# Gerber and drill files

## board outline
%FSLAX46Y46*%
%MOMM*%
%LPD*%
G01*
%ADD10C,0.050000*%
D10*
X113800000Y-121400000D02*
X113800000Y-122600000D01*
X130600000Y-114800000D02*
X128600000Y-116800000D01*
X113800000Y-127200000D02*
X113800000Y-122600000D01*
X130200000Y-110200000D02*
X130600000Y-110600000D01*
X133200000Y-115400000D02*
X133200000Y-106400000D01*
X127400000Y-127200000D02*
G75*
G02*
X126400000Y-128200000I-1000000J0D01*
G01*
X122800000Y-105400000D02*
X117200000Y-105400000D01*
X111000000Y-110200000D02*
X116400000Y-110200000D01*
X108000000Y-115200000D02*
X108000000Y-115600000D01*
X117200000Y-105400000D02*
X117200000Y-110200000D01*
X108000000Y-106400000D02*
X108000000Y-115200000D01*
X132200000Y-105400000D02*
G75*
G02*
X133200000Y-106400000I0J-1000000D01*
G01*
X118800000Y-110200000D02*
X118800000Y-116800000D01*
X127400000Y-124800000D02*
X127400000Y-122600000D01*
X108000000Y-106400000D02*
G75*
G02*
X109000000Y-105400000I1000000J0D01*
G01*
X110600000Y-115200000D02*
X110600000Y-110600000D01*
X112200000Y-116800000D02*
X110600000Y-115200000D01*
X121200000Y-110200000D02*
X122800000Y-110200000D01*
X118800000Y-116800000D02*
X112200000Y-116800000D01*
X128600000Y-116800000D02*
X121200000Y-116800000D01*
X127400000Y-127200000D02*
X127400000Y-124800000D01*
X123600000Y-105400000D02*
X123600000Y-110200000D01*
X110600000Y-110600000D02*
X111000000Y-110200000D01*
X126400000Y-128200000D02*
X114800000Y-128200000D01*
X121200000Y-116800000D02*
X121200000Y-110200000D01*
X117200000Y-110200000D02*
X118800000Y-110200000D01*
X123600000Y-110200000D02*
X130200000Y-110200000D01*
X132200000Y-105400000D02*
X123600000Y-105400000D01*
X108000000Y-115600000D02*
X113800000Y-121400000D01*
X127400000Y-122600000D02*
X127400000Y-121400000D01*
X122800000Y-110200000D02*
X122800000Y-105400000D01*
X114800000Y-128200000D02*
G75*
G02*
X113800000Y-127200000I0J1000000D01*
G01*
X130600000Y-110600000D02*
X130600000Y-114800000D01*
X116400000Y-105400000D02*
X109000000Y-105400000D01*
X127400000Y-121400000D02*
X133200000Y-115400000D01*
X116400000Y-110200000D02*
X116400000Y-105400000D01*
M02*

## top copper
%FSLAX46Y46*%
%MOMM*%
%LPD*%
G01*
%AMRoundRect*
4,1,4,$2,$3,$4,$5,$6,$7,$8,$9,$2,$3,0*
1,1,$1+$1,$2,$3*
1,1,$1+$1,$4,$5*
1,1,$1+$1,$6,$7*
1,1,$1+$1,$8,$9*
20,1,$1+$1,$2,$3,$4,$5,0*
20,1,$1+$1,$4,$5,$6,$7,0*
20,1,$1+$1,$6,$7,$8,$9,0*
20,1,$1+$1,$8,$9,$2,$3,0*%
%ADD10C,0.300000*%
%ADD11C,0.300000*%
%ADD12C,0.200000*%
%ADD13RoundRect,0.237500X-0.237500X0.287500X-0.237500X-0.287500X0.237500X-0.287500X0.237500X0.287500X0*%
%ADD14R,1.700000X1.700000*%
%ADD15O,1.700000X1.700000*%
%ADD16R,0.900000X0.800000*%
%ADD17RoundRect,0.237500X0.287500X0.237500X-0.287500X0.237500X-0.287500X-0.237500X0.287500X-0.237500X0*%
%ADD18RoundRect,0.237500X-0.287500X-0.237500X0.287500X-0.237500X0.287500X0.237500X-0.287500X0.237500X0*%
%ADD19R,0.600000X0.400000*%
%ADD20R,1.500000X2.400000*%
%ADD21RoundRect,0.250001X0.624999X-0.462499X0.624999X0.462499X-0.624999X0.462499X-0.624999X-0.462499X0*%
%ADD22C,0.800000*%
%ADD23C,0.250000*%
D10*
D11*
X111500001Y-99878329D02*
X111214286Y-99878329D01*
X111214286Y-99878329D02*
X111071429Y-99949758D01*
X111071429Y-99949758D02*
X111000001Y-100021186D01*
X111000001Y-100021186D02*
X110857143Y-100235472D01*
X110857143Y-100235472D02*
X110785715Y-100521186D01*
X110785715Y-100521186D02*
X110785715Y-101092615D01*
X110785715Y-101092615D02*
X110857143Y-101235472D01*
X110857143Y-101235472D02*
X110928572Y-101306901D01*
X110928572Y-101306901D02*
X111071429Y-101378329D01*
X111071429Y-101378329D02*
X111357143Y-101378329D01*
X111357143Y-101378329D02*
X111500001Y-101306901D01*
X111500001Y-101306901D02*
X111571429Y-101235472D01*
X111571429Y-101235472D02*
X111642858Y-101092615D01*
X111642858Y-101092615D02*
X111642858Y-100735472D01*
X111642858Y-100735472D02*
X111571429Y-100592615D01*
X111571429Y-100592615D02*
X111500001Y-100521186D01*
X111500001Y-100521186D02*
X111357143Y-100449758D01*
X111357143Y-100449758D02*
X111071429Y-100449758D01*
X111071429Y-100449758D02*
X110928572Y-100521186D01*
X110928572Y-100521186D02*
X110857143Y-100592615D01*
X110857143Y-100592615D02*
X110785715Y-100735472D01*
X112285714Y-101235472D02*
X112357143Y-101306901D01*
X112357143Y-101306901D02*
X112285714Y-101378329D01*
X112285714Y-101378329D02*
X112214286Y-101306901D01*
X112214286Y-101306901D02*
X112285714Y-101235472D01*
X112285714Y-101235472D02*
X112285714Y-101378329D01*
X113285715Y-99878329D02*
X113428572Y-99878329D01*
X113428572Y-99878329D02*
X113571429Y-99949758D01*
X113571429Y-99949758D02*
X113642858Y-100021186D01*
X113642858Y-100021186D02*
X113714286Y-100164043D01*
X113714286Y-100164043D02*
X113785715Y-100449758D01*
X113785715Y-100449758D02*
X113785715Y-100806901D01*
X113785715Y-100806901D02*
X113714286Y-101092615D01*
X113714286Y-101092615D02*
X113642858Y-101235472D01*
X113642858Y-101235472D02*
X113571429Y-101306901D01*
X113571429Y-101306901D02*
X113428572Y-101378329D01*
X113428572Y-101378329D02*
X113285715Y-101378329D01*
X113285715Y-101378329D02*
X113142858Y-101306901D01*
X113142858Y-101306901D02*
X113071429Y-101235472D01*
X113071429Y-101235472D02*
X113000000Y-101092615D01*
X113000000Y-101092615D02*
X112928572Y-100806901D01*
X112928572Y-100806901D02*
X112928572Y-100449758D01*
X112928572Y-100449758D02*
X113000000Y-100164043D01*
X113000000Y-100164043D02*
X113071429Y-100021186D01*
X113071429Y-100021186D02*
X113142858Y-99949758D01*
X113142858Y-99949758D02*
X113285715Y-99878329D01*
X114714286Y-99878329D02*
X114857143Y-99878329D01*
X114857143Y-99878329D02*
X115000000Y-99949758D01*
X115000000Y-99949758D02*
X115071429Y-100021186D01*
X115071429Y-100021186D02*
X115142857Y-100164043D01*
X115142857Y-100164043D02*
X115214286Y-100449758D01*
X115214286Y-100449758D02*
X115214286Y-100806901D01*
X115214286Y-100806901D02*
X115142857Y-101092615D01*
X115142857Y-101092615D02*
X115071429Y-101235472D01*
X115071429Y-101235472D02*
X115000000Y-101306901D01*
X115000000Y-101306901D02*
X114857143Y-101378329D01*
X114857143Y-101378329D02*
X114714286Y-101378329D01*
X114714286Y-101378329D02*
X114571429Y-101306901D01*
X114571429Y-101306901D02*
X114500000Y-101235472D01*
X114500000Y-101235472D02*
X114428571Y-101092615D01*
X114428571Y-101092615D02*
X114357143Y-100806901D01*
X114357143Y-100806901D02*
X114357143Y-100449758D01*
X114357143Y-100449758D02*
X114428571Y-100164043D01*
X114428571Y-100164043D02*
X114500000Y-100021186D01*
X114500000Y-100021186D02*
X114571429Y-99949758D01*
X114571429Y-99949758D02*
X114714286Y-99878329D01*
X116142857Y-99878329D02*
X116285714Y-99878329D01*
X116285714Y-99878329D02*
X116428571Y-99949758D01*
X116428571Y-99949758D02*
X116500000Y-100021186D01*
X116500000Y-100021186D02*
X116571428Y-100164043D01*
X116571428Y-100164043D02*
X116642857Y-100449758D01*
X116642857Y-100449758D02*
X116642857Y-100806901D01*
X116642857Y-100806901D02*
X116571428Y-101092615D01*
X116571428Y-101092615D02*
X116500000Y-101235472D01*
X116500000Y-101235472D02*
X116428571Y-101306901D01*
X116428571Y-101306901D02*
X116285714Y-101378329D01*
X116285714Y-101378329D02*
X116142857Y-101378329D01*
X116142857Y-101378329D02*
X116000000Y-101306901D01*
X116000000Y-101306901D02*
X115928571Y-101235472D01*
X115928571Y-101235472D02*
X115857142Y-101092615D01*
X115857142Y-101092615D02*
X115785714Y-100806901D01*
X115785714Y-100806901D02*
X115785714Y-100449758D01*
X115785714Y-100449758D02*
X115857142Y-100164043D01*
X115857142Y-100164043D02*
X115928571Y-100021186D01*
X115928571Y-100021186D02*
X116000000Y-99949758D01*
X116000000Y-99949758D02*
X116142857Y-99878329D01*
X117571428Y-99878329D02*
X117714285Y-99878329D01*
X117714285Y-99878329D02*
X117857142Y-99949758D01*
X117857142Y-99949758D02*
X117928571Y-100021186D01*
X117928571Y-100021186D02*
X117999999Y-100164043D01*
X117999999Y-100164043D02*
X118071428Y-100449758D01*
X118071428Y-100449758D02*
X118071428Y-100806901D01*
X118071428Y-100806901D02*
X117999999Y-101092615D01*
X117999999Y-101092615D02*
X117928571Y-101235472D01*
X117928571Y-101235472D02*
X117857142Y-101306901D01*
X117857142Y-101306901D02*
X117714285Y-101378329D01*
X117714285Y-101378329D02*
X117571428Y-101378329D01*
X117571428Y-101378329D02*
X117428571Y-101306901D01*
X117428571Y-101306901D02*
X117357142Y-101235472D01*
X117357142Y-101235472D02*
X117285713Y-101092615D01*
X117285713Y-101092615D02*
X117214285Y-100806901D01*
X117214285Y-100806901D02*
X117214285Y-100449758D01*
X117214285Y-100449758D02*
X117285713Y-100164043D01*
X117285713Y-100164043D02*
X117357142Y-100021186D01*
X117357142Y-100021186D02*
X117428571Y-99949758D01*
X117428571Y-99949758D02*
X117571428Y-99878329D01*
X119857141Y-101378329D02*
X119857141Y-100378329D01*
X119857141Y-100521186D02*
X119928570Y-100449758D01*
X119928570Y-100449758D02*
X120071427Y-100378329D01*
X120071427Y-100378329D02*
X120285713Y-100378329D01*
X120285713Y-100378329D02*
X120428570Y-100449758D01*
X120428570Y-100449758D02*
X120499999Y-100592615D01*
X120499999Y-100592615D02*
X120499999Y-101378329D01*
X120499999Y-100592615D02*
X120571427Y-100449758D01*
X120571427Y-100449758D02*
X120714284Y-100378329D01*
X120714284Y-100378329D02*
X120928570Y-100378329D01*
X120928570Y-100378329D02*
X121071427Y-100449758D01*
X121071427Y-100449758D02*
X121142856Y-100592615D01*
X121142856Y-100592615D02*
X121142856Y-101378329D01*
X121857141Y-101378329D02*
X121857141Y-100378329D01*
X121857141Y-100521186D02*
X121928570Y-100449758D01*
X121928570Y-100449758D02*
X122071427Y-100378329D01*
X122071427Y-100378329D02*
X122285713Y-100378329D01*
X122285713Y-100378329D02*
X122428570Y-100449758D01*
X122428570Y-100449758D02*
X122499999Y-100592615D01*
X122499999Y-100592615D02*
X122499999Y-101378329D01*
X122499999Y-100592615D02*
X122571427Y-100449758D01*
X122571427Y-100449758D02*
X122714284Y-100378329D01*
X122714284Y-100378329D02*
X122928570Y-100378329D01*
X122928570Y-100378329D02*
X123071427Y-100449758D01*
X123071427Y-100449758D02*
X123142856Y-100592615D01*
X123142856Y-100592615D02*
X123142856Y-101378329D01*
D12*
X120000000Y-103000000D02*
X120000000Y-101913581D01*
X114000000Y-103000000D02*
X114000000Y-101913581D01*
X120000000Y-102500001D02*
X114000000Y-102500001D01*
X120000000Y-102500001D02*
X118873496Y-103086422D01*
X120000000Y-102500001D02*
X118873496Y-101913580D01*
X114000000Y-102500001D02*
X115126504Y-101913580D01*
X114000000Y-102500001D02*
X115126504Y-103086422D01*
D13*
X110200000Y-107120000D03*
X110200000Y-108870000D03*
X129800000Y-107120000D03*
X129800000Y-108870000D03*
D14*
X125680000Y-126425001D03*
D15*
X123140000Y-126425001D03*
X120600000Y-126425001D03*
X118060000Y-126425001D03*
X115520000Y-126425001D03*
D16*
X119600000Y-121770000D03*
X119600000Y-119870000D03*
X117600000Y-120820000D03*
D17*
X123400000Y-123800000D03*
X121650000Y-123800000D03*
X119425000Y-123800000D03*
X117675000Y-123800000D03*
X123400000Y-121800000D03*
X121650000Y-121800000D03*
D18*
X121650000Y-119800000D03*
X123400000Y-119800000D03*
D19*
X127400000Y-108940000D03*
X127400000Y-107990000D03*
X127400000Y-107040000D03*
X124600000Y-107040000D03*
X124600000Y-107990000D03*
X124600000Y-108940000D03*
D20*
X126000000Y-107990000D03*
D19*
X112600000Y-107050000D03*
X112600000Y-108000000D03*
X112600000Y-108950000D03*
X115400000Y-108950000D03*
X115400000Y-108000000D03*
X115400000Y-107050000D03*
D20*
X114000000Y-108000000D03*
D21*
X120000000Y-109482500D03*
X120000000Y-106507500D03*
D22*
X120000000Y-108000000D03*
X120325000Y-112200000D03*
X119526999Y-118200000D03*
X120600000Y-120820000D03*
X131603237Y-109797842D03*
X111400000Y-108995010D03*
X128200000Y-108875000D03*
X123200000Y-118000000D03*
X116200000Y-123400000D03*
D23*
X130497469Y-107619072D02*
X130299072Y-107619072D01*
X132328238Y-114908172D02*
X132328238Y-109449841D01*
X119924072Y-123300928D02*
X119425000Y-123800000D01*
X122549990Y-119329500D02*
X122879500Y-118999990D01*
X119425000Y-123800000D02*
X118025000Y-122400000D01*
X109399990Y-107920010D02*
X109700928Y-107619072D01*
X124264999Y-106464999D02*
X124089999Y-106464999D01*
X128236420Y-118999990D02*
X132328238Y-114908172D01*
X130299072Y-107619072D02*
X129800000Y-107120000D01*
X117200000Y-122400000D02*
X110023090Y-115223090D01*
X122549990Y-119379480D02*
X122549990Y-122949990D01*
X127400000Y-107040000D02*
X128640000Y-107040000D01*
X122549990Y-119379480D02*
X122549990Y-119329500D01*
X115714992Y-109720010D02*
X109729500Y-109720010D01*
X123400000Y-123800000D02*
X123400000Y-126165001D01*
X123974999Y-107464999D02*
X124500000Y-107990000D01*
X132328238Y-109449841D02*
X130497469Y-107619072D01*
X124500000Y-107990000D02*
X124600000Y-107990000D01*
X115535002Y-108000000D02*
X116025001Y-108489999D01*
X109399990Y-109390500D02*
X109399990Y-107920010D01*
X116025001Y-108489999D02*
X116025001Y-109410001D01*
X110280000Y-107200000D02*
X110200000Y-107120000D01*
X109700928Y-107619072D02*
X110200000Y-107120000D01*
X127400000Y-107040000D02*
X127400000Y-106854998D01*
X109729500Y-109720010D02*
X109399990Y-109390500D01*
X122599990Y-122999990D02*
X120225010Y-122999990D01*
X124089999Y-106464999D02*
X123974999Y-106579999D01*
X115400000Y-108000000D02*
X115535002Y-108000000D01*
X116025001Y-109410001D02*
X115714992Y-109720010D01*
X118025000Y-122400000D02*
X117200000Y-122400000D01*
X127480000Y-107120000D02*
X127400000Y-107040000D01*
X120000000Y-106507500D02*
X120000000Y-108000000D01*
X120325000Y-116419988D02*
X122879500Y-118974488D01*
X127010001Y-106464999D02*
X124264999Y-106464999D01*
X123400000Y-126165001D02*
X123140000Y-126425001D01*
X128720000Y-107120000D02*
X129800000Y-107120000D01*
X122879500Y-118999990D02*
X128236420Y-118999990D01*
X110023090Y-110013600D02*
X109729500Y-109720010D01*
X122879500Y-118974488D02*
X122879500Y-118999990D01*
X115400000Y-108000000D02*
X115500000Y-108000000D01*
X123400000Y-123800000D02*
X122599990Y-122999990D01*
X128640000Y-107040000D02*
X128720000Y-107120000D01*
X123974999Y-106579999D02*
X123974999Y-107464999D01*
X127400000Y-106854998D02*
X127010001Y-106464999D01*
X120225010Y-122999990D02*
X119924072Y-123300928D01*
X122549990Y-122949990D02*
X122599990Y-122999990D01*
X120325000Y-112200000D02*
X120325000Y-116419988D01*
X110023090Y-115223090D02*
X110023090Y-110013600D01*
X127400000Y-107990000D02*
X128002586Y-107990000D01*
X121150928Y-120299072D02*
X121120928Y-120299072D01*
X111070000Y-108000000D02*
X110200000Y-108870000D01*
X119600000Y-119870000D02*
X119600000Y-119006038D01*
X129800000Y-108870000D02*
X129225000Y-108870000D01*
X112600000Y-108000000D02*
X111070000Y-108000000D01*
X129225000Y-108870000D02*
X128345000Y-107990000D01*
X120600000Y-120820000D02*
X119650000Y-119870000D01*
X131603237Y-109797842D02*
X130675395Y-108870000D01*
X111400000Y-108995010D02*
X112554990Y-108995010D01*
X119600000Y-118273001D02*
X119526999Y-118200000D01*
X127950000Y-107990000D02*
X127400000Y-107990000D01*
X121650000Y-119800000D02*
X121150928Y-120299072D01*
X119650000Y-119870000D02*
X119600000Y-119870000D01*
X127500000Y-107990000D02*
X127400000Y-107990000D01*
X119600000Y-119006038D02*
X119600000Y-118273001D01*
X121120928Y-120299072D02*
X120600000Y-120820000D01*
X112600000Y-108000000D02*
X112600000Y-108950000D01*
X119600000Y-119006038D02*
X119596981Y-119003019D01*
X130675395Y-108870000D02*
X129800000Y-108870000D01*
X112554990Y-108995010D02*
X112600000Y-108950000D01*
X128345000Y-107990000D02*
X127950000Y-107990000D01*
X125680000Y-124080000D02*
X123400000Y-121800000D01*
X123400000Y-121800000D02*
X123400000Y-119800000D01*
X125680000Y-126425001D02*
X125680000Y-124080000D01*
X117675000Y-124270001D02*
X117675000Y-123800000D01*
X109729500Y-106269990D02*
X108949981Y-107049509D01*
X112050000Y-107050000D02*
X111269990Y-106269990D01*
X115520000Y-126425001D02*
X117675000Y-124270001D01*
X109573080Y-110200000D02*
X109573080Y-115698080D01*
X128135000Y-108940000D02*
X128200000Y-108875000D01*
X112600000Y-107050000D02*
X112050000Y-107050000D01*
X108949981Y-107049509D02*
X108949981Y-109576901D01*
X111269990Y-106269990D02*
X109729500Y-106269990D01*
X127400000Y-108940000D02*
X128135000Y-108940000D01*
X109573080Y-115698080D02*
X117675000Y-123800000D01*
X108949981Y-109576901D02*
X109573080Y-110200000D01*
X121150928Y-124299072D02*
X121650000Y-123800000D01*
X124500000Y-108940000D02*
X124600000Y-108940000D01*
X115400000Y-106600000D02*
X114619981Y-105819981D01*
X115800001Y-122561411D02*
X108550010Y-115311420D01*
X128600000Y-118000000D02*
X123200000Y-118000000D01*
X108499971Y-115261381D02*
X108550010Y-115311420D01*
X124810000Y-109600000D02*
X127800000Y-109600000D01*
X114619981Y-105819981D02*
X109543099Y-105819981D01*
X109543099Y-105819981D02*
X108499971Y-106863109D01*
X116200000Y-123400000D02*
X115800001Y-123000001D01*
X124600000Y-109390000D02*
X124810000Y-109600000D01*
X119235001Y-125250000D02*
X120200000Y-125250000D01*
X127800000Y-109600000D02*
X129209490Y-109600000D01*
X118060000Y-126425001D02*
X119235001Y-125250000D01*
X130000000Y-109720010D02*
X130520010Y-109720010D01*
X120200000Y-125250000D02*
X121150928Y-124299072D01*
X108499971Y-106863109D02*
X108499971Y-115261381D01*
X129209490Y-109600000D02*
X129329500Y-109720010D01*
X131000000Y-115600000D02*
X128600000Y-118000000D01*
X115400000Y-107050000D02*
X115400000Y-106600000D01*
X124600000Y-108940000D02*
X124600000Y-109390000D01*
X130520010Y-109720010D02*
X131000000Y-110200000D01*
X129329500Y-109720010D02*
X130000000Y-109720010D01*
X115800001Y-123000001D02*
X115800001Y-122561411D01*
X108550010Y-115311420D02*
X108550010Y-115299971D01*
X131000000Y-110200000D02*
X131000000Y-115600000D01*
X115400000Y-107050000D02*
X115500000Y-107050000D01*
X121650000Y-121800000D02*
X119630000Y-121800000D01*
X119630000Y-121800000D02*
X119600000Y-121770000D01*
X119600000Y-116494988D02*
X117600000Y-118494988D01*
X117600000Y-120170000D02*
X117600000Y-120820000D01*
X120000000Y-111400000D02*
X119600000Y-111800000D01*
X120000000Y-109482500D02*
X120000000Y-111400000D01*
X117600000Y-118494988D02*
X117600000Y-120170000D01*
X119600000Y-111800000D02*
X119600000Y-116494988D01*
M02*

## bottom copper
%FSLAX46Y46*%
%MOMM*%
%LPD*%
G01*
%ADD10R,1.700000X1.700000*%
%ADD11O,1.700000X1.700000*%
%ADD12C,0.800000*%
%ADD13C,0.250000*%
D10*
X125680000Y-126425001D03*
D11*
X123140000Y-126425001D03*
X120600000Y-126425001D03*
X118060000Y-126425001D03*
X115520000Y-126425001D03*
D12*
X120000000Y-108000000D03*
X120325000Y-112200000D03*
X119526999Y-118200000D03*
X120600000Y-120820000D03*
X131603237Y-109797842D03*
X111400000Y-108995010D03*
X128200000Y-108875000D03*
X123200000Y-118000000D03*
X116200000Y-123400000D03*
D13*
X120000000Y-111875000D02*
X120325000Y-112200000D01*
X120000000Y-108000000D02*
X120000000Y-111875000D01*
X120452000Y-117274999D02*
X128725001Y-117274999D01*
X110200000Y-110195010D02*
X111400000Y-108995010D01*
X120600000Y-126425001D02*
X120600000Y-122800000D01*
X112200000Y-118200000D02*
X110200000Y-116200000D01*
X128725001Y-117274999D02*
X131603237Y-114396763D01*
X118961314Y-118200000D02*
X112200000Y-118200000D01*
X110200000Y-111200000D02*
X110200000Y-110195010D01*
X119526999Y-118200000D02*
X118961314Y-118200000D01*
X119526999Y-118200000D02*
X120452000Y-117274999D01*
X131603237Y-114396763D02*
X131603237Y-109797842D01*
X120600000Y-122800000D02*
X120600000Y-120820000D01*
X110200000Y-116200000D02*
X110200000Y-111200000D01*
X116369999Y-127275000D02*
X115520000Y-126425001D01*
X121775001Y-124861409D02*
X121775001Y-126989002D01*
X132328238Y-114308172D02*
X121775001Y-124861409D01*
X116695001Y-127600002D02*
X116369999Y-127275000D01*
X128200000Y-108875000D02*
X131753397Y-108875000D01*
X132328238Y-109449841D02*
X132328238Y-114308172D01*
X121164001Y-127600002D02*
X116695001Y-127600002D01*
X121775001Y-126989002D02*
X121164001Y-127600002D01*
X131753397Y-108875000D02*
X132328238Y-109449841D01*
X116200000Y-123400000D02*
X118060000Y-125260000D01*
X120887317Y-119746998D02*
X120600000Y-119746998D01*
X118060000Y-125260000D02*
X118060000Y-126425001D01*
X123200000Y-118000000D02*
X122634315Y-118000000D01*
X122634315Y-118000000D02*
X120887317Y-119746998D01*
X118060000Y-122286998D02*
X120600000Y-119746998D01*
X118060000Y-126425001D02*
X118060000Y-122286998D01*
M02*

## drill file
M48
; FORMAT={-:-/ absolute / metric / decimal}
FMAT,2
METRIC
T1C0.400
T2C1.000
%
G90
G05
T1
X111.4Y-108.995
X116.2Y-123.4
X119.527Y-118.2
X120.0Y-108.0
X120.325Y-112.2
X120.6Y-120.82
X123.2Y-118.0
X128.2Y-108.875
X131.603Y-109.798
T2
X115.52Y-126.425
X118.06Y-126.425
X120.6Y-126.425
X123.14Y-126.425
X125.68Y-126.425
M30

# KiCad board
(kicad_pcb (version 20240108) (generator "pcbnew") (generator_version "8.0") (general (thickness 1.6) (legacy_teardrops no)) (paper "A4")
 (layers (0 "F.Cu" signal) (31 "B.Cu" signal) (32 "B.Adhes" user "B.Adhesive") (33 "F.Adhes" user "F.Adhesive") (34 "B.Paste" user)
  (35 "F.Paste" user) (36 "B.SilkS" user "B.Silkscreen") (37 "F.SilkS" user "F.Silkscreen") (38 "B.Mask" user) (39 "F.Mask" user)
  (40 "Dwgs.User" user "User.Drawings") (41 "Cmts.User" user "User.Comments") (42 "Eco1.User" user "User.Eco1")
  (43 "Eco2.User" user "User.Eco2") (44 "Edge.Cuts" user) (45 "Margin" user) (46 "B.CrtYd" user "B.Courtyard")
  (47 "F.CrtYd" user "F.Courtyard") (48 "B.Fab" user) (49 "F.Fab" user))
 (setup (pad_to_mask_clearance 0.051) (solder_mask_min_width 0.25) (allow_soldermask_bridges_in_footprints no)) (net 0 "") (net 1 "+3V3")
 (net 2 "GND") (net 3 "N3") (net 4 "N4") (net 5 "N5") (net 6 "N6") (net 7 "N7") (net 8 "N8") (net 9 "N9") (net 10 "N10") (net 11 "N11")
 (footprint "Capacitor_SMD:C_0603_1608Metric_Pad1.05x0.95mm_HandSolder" (layer "F.Cu") (at 110.2 107.995 -90)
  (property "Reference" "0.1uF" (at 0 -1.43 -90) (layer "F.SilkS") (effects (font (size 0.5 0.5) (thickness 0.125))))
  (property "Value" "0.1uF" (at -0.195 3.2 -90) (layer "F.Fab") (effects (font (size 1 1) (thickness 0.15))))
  (pad "1" smd roundrect (at -0.875 0 270) (size 1.05 0.95) (layers "F.Cu" "F.Paste" "F.Mask") (roundrect_rratio 0.25) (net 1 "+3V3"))
  (pad "2" smd roundrect (at 0.875 0 270) (size 1.05 0.95) (layers "F.Cu" "F.Paste" "F.Mask") (roundrect_rratio 0.25) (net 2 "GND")))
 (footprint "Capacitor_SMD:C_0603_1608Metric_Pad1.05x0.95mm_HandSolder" (layer "F.Cu") (at 129.8 107.995 -90)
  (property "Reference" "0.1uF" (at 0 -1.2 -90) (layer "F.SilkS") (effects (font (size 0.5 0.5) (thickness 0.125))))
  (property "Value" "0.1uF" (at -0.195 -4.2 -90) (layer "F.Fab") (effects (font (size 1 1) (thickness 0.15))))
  (pad "1" smd roundrect (at -0.875 0 270) (size 1.05 0.95) (layers "F.Cu" "F.Paste" "F.Mask") (roundrect_rratio 0.25) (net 1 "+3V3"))
  (pad "2" smd roundrect (at 0.875 0 270) (size 1.05 0.95) (layers "F.Cu" "F.Paste" "F.Mask") (roundrect_rratio 0.25) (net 2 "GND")))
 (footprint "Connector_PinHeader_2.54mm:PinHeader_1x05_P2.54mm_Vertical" (layer "F.Cu") (at 125.68 126.425001 -90)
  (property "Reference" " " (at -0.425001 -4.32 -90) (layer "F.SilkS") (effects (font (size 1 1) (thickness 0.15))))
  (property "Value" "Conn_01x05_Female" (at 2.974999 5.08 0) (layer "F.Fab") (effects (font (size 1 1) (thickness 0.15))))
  (pad "1" thru_hole rect (at 0 0 270) (size 1.7 1.7) (drill 1) (layers "*.Cu" "*.Mask") (remove_unused_layers no) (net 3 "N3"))
  (pad "2" thru_hole oval (at 0 2.54 270) (size 1.7 1.7) (drill 1) (layers "*.Cu" "*.Mask") (remove_unused_layers no) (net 1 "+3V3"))
  (pad "3" thru_hole oval (at 0 5.08 270) (size 1.7 1.7) (drill 1) (layers "*.Cu" "*.Mask") (remove_unused_layers no) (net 2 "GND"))
  (pad "4" thru_hole oval (at 0 7.62 270) (size 1.7 1.7) (drill 1) (layers "*.Cu" "*.Mask") (remove_unused_layers no) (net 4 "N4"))
  (pad "5" thru_hole oval (at 0 10.16 270) (size 1.7 1.7) (drill 1) (layers "*.Cu" "*.Mask") (remove_unused_layers no) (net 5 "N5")))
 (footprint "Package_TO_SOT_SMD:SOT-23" (layer "F.Cu") (at 118.6 120.82 180)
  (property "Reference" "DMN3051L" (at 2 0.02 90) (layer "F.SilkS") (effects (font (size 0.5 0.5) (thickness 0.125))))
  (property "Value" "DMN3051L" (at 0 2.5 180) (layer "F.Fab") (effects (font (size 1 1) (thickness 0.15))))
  (pad "1" smd rect (at -1 -0.95 180) (size 0.9 0.8) (layers "F.Cu" "F.Paste" "F.Mask") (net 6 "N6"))
  (pad "2" smd rect (at -1 0.95 180) (size 0.9 0.8) (layers "F.Cu" "F.Paste" "F.Mask") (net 2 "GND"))
  (pad "3" smd rect (at 1 0 180) (size 0.9 0.8) (layers "F.Cu" "F.Paste" "F.Mask") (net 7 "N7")))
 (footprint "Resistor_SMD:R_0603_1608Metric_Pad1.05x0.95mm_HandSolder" (layer "F.Cu") (at 122.525 123.8 180)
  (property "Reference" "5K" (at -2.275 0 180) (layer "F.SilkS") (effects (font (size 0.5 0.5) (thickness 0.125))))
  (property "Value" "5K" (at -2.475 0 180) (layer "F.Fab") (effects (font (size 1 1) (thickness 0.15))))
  (pad "1" smd roundrect (at -0.875 0 180) (size 1.05 0.95) (layers "F.Cu" "F.Paste" "F.Mask") (roundrect_rratio 0.25) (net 1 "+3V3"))
  (pad "2" smd roundrect (at 0.875 0 180) (size 1.05 0.95) (layers "F.Cu" "F.Paste" "F.Mask") (roundrect_rratio 0.25) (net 4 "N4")))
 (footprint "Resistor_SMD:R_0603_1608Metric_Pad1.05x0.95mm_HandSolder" (layer "F.Cu") (at 118.55 123.8 180)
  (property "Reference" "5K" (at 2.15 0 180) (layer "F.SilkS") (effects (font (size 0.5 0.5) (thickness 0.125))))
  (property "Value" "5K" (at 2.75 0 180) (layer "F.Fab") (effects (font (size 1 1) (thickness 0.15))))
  (pad "1" smd roundrect (at -0.875 0 180) (size 1.05 0.95) (layers "F.Cu" "F.Paste" "F.Mask") (roundrect_rratio 0.25) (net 1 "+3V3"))
  (pad "2" smd roundrect (at 0.875 0 180) (size 1.05 0.95) (layers "F.Cu" "F.Paste" "F.Mask") (roundrect_rratio 0.25) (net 5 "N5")))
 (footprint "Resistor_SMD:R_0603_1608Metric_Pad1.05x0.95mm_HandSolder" (layer "F.Cu") (at 122.525 121.8 180)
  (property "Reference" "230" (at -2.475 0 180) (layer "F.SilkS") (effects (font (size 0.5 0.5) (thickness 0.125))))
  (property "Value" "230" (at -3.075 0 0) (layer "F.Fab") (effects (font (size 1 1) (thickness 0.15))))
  (pad "1" smd roundrect (at -0.875 0 180) (size 1.05 0.95) (layers "F.Cu" "F.Paste" "F.Mask") (roundrect_rratio 0.25) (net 3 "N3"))
  (pad "2" smd roundrect (at 0.875 0 180) (size 1.05 0.95) (layers "F.Cu" "F.Paste" "F.Mask") (roundrect_rratio 0.25) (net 6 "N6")))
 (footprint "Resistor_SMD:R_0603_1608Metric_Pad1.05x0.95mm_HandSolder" (layer "F.Cu") (at 122.525 119.8)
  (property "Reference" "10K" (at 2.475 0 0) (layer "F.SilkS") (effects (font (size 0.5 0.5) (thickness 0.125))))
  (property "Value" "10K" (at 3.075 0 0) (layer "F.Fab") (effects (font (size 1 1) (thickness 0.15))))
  (pad "1" smd roundrect (at -0.875 0) (size 1.05 0.95) (layers "F.Cu" "F.Paste" "F.Mask") (roundrect_rratio 0.25) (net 2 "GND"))
  (pad "2" smd roundrect (at 0.875 0) (size 1.05 0.95) (layers "F.Cu" "F.Paste" "F.Mask") (roundrect_rratio 0.25) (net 3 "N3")))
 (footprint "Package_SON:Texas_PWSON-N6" (layer "F.Cu") (at 126 107.99 180)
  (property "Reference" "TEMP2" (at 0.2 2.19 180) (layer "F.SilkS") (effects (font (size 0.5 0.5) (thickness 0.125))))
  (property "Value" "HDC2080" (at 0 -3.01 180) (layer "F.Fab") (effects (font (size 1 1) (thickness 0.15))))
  (pad "1" smd rect (at -1.4 -0.95 180) (size 0.6 0.4) (layers "F.Cu" "F.Paste" "F.Mask") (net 5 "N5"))
  (pad "2" smd rect (at -1.4 0 180) (size 0.6 0.4) (layers "F.Cu" "F.Paste" "F.Mask") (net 2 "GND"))
  (pad "3" smd rect (at -1.4 0.95 180) (size 0.6 0.4) (layers "F.Cu" "F.Paste" "F.Mask") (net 1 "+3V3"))
  (pad "4" smd rect (at 1.4 0.95 180) (size 0.6 0.4) (layers "F.Cu" "F.Paste" "F.Mask") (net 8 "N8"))
  (pad "5" smd rect (at 1.4 0 180) (size 0.6 0.4) (layers "F.Cu" "F.Paste" "F.Mask") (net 1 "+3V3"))
  (pad "6" smd rect (at 1.4 -0.95 180) (size 0.6 0.4) (layers "F.Cu" "F.Paste" "F.Mask") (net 4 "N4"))
  (pad "7" smd rect (at 0 0 180) (size 1.5 2.4) (layers "F.Cu" "F.Paste" "F.Mask") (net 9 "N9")))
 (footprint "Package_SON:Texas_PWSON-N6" (layer "F.Cu") (at 114 108)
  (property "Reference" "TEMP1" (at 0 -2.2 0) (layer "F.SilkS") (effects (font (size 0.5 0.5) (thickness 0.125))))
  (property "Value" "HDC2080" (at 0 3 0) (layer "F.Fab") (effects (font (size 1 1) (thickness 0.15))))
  (pad "1" smd rect (at -1.4 -0.95) (size 0.6 0.4) (layers "F.Cu" "F.Paste" "F.Mask") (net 5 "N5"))
  (pad "2" smd rect (at -1.4 0) (size 0.6 0.4) (layers "F.Cu" "F.Paste" "F.Mask") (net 2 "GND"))
  (pad "3" smd rect (at -1.4 0.95) (size 0.6 0.4) (layers "F.Cu" "F.Paste" "F.Mask") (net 2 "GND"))
  (pad "4" smd rect (at 1.4 0.95) (size 0.6 0.4) (layers "F.Cu" "F.Paste" "F.Mask") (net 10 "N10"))
  (pad "5" smd rect (at 1.4 0) (size 0.6 0.4) (layers "F.Cu" "F.Paste" "F.Mask") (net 1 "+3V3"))
  (pad "6" smd rect (at 1.4 -0.95) (size 0.6 0.4) (layers "F.Cu" "F.Paste" "F.Mask") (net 4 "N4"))
  (pad "7" smd rect (at 0 0) (size 1.5 2.4) (layers "F.Cu" "F.Paste" "F.Mask") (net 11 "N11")))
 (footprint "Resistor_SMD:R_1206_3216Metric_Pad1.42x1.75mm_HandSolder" (layer "F.Cu") (at 120 107.995 90)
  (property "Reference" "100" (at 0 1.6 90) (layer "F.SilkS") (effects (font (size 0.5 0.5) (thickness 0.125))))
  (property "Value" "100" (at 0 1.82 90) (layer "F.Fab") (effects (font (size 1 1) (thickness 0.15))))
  (pad "1" smd roundrect (at -1.4875 0 90) (size 1.425 1.75) (layers "F.Cu" "F.Paste" "F.Mask") (roundrect_rratio 0.175439) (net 7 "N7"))
  (pad "2" smd roundrect (at 1.4875 0 90) (size 1.425 1.75) (layers "F.Cu" "F.Paste" "F.Mask") (roundrect_rratio 0.175439) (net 1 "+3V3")))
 (gr_line (start 113.8 121.4) (end 113.8 122.6) (stroke (width 0.05) (type solid)) (layer "Edge.Cuts"))
 (gr_line (start 130.6 114.8) (end 128.6 116.8) (stroke (width 0.05) (type solid)) (layer "Edge.Cuts"))
 (gr_line (start 113.8 127.2) (end 113.8 122.6) (stroke (width 0.05) (type solid)) (layer "Edge.Cuts"))
 (gr_line (start 130.2 110.2) (end 130.6 110.6) (stroke (width 0.05) (type solid)) (layer "Edge.Cuts"))
 (gr_line (start 133.2 115.4) (end 133.2 106.4) (stroke (width 0.05) (type solid)) (layer "Edge.Cuts"))
 (gr_arc (start 127.4 127.2) (mid 127.107107 127.907107) (end 126.4 128.2) (stroke (width 0.05) (type solid)) (layer "Edge.Cuts"))
 (gr_line (start 122.8 105.4) (end 117.2 105.4) (stroke (width 0.05) (type solid)) (layer "Edge.Cuts"))
 (gr_line (start 111 110.2) (end 116.4 110.2) (stroke (width 0.05) (type solid)) (layer "Edge.Cuts"))
 (gr_line (start 108 115.2) (end 108 115.6) (stroke (width 0.05) (type solid)) (layer "Edge.Cuts"))
 (gr_line (start 117.2 105.4) (end 117.2 110.2) (stroke (width 0.05) (type solid)) (layer "Edge.Cuts"))
 (gr_line (start 108 106.4) (end 108 115.2) (stroke (width 0.05) (type solid)) (layer "Edge.Cuts"))
 (gr_arc (start 132.2 105.4) (mid 132.907107 105.692893) (end 133.2 106.4) (stroke (width 0.05) (type solid)) (layer "Edge.Cuts"))
 (gr_line (start 118.8 110.2) (end 118.8 116.8) (stroke (width 0.05) (type solid)) (layer "Edge.Cuts"))
 (gr_line (start 127.4 124.8) (end 127.4 122.6) (stroke (width 0.05) (type solid)) (layer "Edge.Cuts"))
 (gr_arc (start 108 106.4) (mid 108.292893 105.692893) (end 109 105.4) (stroke (width 0.05) (type solid)) (layer "Edge.Cuts"))
 (gr_line (start 110.6 115.2) (end 110.6 110.6) (stroke (width 0.05) (type solid)) (layer "Edge.Cuts"))
 (gr_line (start 112.2 116.8) (end 110.6 115.2) (stroke (width 0.05) (type solid)) (layer "Edge.Cuts"))
 (gr_line (start 121.2 110.2) (end 122.8 110.2) (stroke (width 0.05) (type solid)) (layer "Edge.Cuts"))
 (gr_line (start 118.8 116.8) (end 112.2 116.8) (stroke (width 0.05) (type solid)) (layer "Edge.Cuts"))
 (gr_line (start 128.6 116.8) (end 121.2 116.8) (stroke (width 0.05) (type solid)) (layer "Edge.Cuts"))
 (gr_line (start 127.4 127.2) (end 127.4 124.8) (stroke (width 0.05) (type solid)) (layer "Edge.Cuts"))
 (gr_line (start 123.6 105.4) (end 123.6 110.2) (stroke (width 0.05) (type solid)) (layer "Edge.Cuts"))
 (gr_line (start 110.6 110.6) (end 111 110.2) (stroke (width 0.05) (type solid)) (layer "Edge.Cuts"))
 (gr_line (start 126.4 128.2) (end 114.8 128.2) (stroke (width 0.05) (type solid)) (layer "Edge.Cuts"))
 (gr_line (start 121.2 116.8) (end 121.2 110.2) (stroke (width 0.05) (type solid)) (layer "Edge.Cuts"))
 (gr_line (start 117.2 110.2) (end 118.8 110.2) (stroke (width 0.05) (type solid)) (layer "Edge.Cuts"))
 (gr_line (start 123.6 110.2) (end 130.2 110.2) (stroke (width 0.05) (type solid)) (layer "Edge.Cuts"))
 (gr_line (start 132.2 105.4) (end 123.6 105.4) (stroke (width 0.05) (type solid)) (layer "Edge.Cuts"))
 (gr_line (start 108 115.6) (end 113.8 121.4) (stroke (width 0.05) (type solid)) (layer "Edge.Cuts"))
 (gr_line (start 127.4 122.6) (end 127.4 121.4) (stroke (width 0.05) (type solid)) (layer "Edge.Cuts"))
 (gr_line (start 122.8 110.2) (end 122.8 105.4) (stroke (width 0.05) (type solid)) (layer "Edge.Cuts"))
 (gr_arc (start 114.8 128.2) (mid 114.092893 127.907107) (end 113.8 127.2) (stroke (width 0.05) (type solid)) (layer "Edge.Cuts"))
 (gr_line (start 130.6 110.6) (end 130.6 114.8) (stroke (width 0.05) (type solid)) (layer "Edge.Cuts"))
 (gr_line (start 116.4 105.4) (end 109 105.4) (stroke (width 0.05) (type solid)) (layer "Edge.Cuts"))
 (gr_line (start 127.4 121.4) (end 133.2 115.4) (stroke (width 0.05) (type solid)) (layer "Edge.Cuts"))
 (gr_line (start 116.4 110.2) (end 116.4 105.4) (stroke (width 0.05) (type solid)) (layer "Edge.Cuts"))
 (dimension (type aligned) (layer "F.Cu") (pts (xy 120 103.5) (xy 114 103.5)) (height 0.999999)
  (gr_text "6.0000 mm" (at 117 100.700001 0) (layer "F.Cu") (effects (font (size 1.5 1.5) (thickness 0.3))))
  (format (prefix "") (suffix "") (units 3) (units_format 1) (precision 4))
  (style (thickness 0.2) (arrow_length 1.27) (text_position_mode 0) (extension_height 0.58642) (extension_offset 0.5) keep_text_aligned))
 (segment (start 130.497469 107.619072) (end 130.299072 107.619072) (width 0.25) (layer "F.Cu") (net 1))
 (segment (start 132.328238 114.908172) (end 132.328238 109.449841) (width 0.25) (layer "F.Cu") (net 1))
 (segment (start 119.924072 123.300928) (end 119.425 123.8) (width 0.25) (layer "F.Cu") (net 1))
 (segment (start 122.54999 119.3295) (end 122.8795 118.99999) (width 0.25) (layer "F.Cu") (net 1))
 (segment (start 119.425 123.8) (end 118.025 122.4) (width 0.25) (layer "F.Cu") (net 1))
 (segment (start 109.39999 107.92001) (end 109.700928 107.619072) (width 0.25) (layer "F.Cu") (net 1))
 (segment (start 124.264999 106.464999) (end 124.089999 106.464999) (width 0.25) (layer "F.Cu") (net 1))
 (segment (start 128.23642 118.99999) (end 132.328238 114.908172) (width 0.25) (layer "F.Cu") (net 1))
 (segment (start 130.299072 107.619072) (end 129.8 107.12) (width 0.25) (layer "F.Cu") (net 1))
 (segment (start 117.2 122.4) (end 110.02309 115.22309) (width 0.25) (layer "F.Cu") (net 1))
 (segment (start 122.54999 119.37948) (end 122.54999 122.94999) (width 0.25) (layer "F.Cu") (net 1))
 (segment (start 127.4 107.04) (end 128.64 107.04) (width 0.25) (layer "F.Cu") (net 1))
 (segment (start 122.54999 119.37948) (end 122.54999 119.3295) (width 0.25) (layer "F.Cu") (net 1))
 (segment (start 115.714992 109.72001) (end 109.7295 109.72001) (width 0.25) (layer "F.Cu") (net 1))
 (segment (start 123.4 123.8) (end 123.4 126.165001) (width 0.25) (layer "F.Cu") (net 1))
 (segment (start 123.974999 107.464999) (end 124.5 107.99) (width 0.25) (layer "F.Cu") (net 1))
 (segment (start 132.328238 109.449841) (end 130.497469 107.619072) (width 0.25) (layer "F.Cu") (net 1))
 (segment (start 124.5 107.99) (end 124.6 107.99) (width 0.25) (layer "F.Cu") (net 1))
 (segment (start 115.535002 108) (end 116.025001 108.489999) (width 0.25) (layer "F.Cu") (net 1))
 (segment (start 109.39999 109.3905) (end 109.39999 107.92001) (width 0.25) (layer "F.Cu") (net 1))
 (segment (start 116.025001 108.489999) (end 116.025001 109.410001) (width 0.25) (layer "F.Cu") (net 1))
 (segment (start 110.28 107.2) (end 110.2 107.12) (width 0.25) (layer "F.Cu") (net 1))
 (segment (start 109.700928 107.619072) (end 110.2 107.12) (width 0.25) (layer "F.Cu") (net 1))
 (segment (start 127.4 107.04) (end 127.4 106.854998) (width 0.25) (layer "F.Cu") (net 1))
 (segment (start 109.7295 109.72001) (end 109.39999 109.3905) (width 0.25) (layer "F.Cu") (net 1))
 (segment (start 122.59999 122.99999) (end 120.22501 122.99999) (width 0.25) (layer "F.Cu") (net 1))
 (segment (start 124.089999 106.464999) (end 123.974999 106.579999) (width 0.25) (layer "F.Cu") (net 1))
 (segment (start 115.4 108) (end 115.535002 108) (width 0.25) (layer "F.Cu") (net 1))
 (segment (start 116.025001 109.410001) (end 115.714992 109.72001) (width 0.25) (layer "F.Cu") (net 1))
 (segment (start 118.025 122.4) (end 117.2 122.4) (width 0.25) (layer "F.Cu") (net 1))
 (segment (start 127.48 107.12) (end 127.4 107.04) (width 0.25) (layer "F.Cu") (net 1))
 (segment (start 120 106.5075) (end 120 108) (width 0.25) (layer "F.Cu") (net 1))
 (segment (start 120.325 116.419988) (end 122.8795 118.974488) (width 0.25) (layer "F.Cu") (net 1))
 (segment (start 127.010001 106.464999) (end 124.264999 106.464999) (width 0.25) (layer "F.Cu") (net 1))
 (segment (start 123.4 126.165001) (end 123.14 126.425001) (width 0.25) (layer "F.Cu") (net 1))
 (segment (start 128.72 107.12) (end 129.8 107.12) (width 0.25) (layer "F.Cu") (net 1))
 (segment (start 122.8795 118.99999) (end 128.23642 118.99999) (width 0.25) (layer "F.Cu") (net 1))
 (segment (start 110.02309 110.0136) (end 109.7295 109.72001) (width 0.25) (layer "F.Cu") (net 1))
 (segment (start 122.8795 118.974488) (end 122.8795 118.99999) (width 0.25) (layer "F.Cu") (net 1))
 (segment (start 115.4 108) (end 115.5 108) (width 0.25) (layer "F.Cu") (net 1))
 (segment (start 123.4 123.8) (end 122.59999 122.99999) (width 0.25) (layer "F.Cu") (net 1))
 (segment (start 128.64 107.04) (end 128.72 107.12) (width 0.25) (layer "F.Cu") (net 1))
 (segment (start 123.974999 106.579999) (end 123.974999 107.464999) (width 0.25) (layer "F.Cu") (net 1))
 (segment (start 127.4 106.854998) (end 127.010001 106.464999) (width 0.25) (layer "F.Cu") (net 1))
 (segment (start 120.22501 122.99999) (end 119.924072 123.300928) (width 0.25) (layer "F.Cu") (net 1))
 (segment (start 122.54999 122.94999) (end 122.59999 122.99999) (width 0.25) (layer "F.Cu") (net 1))
 (segment (start 120.325 112.2) (end 120.325 116.419988) (width 0.25) (layer "F.Cu") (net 1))
 (segment (start 110.02309 115.22309) (end 110.02309 110.0136) (width 0.25) (layer "F.Cu") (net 1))
 (via (at 120 108) (size 0.8) (drill 0.4) (layers "F.Cu" "B.Cu") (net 1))
 (via (at 120.325 112.2) (size 0.8) (drill 0.4) (layers "F.Cu" "B.Cu") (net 1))
 (segment (start 120 111.875) (end 120.325 112.2) (width 0.25) (layer "B.Cu") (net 1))
 (segment (start 120 108) (end 120 111.875) (width 0.25) (layer "B.Cu") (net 1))
 (segment (start 127.4 107.99) (end 128.002586 107.99) (width 0.25) (layer "F.Cu") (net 2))
 (segment (start 121.150928 120.299072) (end 121.120928 120.299072) (width 0.25) (layer "F.Cu") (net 2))
 (segment (start 111.07 108) (end 110.2 108.87) (width 0.25) (layer "F.Cu") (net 2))
 (segment (start 119.6 119.87) (end 119.6 119.006038) (width 0.25) (layer "F.Cu") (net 2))
 (segment (start 129.8 108.87) (end 129.225 108.87) (width 0.25) (layer "F.Cu") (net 2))
 (segment (start 112.6 108) (end 111.07 108) (width 0.25) (layer "F.Cu") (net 2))
 (segment (start 129.225 108.87) (end 128.345 107.99) (width 0.25) (layer "F.Cu") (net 2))
 (segment (start 120.6 120.82) (end 119.65 119.87) (width 0.25) (layer "F.Cu") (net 2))
 (segment (start 131.603237 109.797842) (end 130.675395 108.87) (width 0.25) (layer "F.Cu") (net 2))
 (segment (start 111.4 108.99501) (end 112.55499 108.99501) (width 0.25) (layer "F.Cu") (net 2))
 (segment (start 119.6 118.273001) (end 119.526999 118.2) (width 0.25) (layer "F.Cu") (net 2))
 (segment (start 127.95 107.99) (end 127.4 107.99) (width 0.25) (layer "F.Cu") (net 2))
 (segment (start 121.65 119.8) (end 121.150928 120.299072) (width 0.25) (layer "F.Cu") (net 2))
 (segment (start 119.65 119.87) (end 119.6 119.87) (width 0.25) (layer "F.Cu") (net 2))
 (segment (start 127.5 107.99) (end 127.4 107.99) (width 0.25) (layer "F.Cu") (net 2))
 (segment (start 119.6 119.006038) (end 119.6 118.273001) (width 0.25) (layer "F.Cu") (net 2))
 (segment (start 121.120928 120.299072) (end 120.6 120.82) (width 0.25) (layer "F.Cu") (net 2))
 (segment (start 112.6 108) (end 112.6 108.95) (width 0.25) (layer "F.Cu") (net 2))
 (segment (start 119.6 119.006038) (end 119.596981 119.003019) (width 0.25) (layer "F.Cu") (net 2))
 (segment (start 130.675395 108.87) (end 129.8 108.87) (width 0.25) (layer "F.Cu") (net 2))
 (segment (start 112.55499 108.99501) (end 112.6 108.95) (width 0.25) (layer "F.Cu") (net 2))
 (segment (start 128.345 107.99) (end 127.95 107.99) (width 0.25) (layer "F.Cu") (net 2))
 (via (at 119.526999 118.2) (size 0.8) (drill 0.4) (layers "F.Cu" "B.Cu") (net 2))
 (via (at 120.6 120.82) (size 0.8) (drill 0.4) (layers "F.Cu" "B.Cu") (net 2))
 (via (at 131.603237 109.797842) (size 0.8) (drill 0.4) (layers "F.Cu" "B.Cu") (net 2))
 (via (at 111.4 108.99501) (size 0.8) (drill 0.4) (layers "F.Cu" "B.Cu") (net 2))
 (segment (start 120.452 117.274999) (end 128.725001 117.274999) (width 0.25) (layer "B.Cu") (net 2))
 (segment (start 110.2 110.19501) (end 111.4 108.99501) (width 0.25) (layer "B.Cu") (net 2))
 (segment (start 120.6 126.425001) (end 120.6 122.8) (width 0.25) (layer "B.Cu") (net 2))
 (segment (start 112.2 118.2) (end 110.2 116.2) (width 0.25) (layer "B.Cu") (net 2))
 (segment (start 128.725001 117.274999) (end 131.603237 114.396763) (width 0.25) (layer "B.Cu") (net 2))
 (segment (start 118.961314 118.2) (end 112.2 118.2) (width 0.25) (layer "B.Cu") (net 2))
 (segment (start 110.2 111.2) (end 110.2 110.19501) (width 0.25) (layer "B.Cu") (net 2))
 (segment (start 119.526999 118.2) (end 118.961314 118.2) (width 0.25) (layer "B.Cu") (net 2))
 (segment (start 119.526999 118.2) (end 120.452 117.274999) (width 0.25) (layer "B.Cu") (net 2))
 (segment (start 131.603237 114.396763) (end 131.603237 109.797842) (width 0.25) (layer "B.Cu") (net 2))
 (segment (start 120.6 122.8) (end 120.6 120.82) (width 0.25) (layer "B.Cu") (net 2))
 (segment (start 110.2 116.2) (end 110.2 111.2) (width 0.25) (layer "B.Cu") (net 2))
 (segment (start 125.68 124.08) (end 123.4 121.8) (width 0.25) (layer "F.Cu") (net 3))
 (segment (start 123.4 121.8) (end 123.4 119.8) (width 0.25) (layer "F.Cu") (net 3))
 (segment (start 125.68 126.425001) (end 125.68 124.08) (width 0.25) (layer "F.Cu") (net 3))
 (segment (start 117.675 124.270001) (end 117.675 123.8) (width 0.25) (layer "F.Cu") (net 5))
 (segment (start 109.7295 106.26999) (end 108.949981 107.049509) (width 0.25) (layer "F.Cu") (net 5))
 (segment (start 112.05 107.05) (end 111.26999 106.26999) (width 0.25) (layer "F.Cu") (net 5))
 (segment (start 115.52 126.425001) (end 117.675 124.270001) (width 0.25) (layer "F.Cu") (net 5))
 (segment (start 109.57308 110.2) (end 109.57308 115.69808) (width 0.25) (layer "F.Cu") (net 5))
 (segment (start 128.135 108.94) (end 128.2 108.875) (width 0.25) (layer "F.Cu") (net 5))
 (segment (start 112.6 107.05) (end 112.05 107.05) (width 0.25) (layer "F.Cu") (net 5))
 (segment (start 108.949981 107.049509) (end 108.949981 109.576901) (width 0.25) (layer "F.Cu") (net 5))
 (segment (start 111.26999 106.26999) (end 109.7295 106.26999) (width 0.25) (layer "F.Cu") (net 5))
 (segment (start 127.4 108.94) (end 128.135 108.94) (width 0.25) (layer "F.Cu") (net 5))
 (segment (start 109.57308 115.69808) (end 117.675 123.8) (width 0.25) (layer "F.Cu") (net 5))
 (segment (start 108.949981 109.576901) (end 109.57308 110.2) (width 0.25) (layer "F.Cu") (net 5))
 (via (at 128.2 108.875) (size 0.8) (drill 0.4) (layers "F.Cu" "B.Cu") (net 5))
 (segment (start 116.369999 127.275) (end 115.52 126.425001) (width 0.25) (layer "B.Cu") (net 5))
 (segment (start 121.775001 124.861409) (end 121.775001 126.989002) (width 0.25) (layer "B.Cu") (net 5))
 (segment (start 132.328238 114.308172) (end 121.775001 124.861409) (width 0.25) (layer "B.Cu") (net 5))
 (segment (start 116.695001 127.600002) (end 116.369999 127.275) (width 0.25) (layer "B.Cu") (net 5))
 (segment (start 128.2 108.875) (end 131.753397 108.875) (width 0.25) (layer "B.Cu") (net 5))
 (segment (start 132.328238 109.449841) (end 132.328238 114.308172) (width 0.25) (layer "B.Cu") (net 5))
 (segment (start 121.164001 127.600002) (end 116.695001 127.600002) (width 0.25) (layer "B.Cu") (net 5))
 (segment (start 121.775001 126.989002) (end 121.164001 127.600002) (width 0.25) (layer "B.Cu") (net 5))
 (segment (start 131.753397 108.875) (end 132.328238 109.449841) (width 0.25) (layer "B.Cu") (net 5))
 (segment (start 121.150928 124.299072) (end 121.65 123.8) (width 0.25) (layer "F.Cu") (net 4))
 (segment (start 124.5 108.94) (end 124.6 108.94) (width 0.25) (layer "F.Cu") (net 4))
 (segment (start 115.4 106.6) (end 114.619981 105.819981) (width 0.25) (layer "F.Cu") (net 4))
 (segment (start 115.800001 122.561411) (end 108.55001 115.31142) (width 0.25) (layer "F.Cu") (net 4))
 (segment (start 128.6 118) (end 123.2 118) (width 0.25) (layer "F.Cu") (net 4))
 (segment (start 108.499971 115.261381) (end 108.55001 115.31142) (width 0.25) (layer "F.Cu") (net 4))
 (segment (start 124.81 109.6) (end 127.8 109.6) (width 0.25) (layer "F.Cu") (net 4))
 (segment (start 114.619981 105.819981) (end 109.543099 105.819981) (width 0.25) (layer "F.Cu") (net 4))
 (segment (start 109.543099 105.819981) (end 108.499971 106.863109) (width 0.25) (layer "F.Cu") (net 4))
 (segment (start 116.2 123.4) (end 115.800001 123.000001) (width 0.25) (layer "F.Cu") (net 4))
 (segment (start 124.6 109.39) (end 124.81 109.6) (width 0.25) (layer "F.Cu") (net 4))
 (segment (start 119.235001 125.25) (end 120.2 125.25) (width 0.25) (layer "F.Cu") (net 4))
 (segment (start 127.8 109.6) (end 129.20949 109.6) (width 0.25) (layer "F.Cu") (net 4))
 (segment (start 118.06 126.425001) (end 119.235001 125.25) (width 0.25) (layer "F.Cu") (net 4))
 (segment (start 130 109.72001) (end 130.52001 109.72001) (width 0.25) (layer "F.Cu") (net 4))
 (segment (start 120.2 125.25) (end 121.150928 124.299072) (width 0.25) (layer "F.Cu") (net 4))
 (segment (start 108.499971 106.863109) (end 108.499971 115.261381) (width 0.25) (layer "F.Cu") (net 4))
 (segment (start 129.20949 109.6) (end 129.3295 109.72001) (width 0.25) (layer "F.Cu") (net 4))
 (segment (start 131 115.6) (end 128.6 118) (width 0.25) (layer "F.Cu") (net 4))
 (segment (start 115.4 107.05) (end 115.4 106.6) (width 0.25) (layer "F.Cu") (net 4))
 (segment (start 124.6 108.94) (end 124.6 109.39) (width 0.25) (layer "F.Cu") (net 4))
 (segment (start 130.52001 109.72001) (end 131 110.2) (width 0.25) (layer "F.Cu") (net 4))
 (segment (start 129.3295 109.72001) (end 130 109.72001) (width 0.25) (layer "F.Cu") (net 4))
 (segment (start 115.800001 123.000001) (end 115.800001 122.561411) (width 0.25) (layer "F.Cu") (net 4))
 (segment (start 108.55001 115.31142) (end 108.55001 115.299971) (width 0.25) (layer "F.Cu") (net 4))
 (segment (start 131 110.2) (end 131 115.6) (width 0.25) (layer "F.Cu") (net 4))
 (segment (start 115.4 107.05) (end 115.5 107.05) (width 0.25) (layer "F.Cu") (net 4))
 (via (at 123.2 118) (size 0.8) (drill 0.4) (layers "F.Cu" "B.Cu") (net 4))
 (via (at 116.2 123.4) (size 0.8) (drill 0.4) (layers "F.Cu" "B.Cu") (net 4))
 (segment (start 116.2 123.4) (end 118.06 125.26) (width 0.25) (layer "B.Cu") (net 4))
 (segment (start 120.887317 119.746998) (end 120.6 119.746998) (width 0.25) (layer "B.Cu") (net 4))
 (segment (start 118.06 125.26) (end 118.06 126.425001) (width 0.25) (layer "B.Cu") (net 4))
 (segment (start 123.2 118) (end 122.634315 118) (width 0.25) (layer "B.Cu") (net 4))
 (segment (start 122.634315 118) (end 120.887317 119.746998) (width 0.25) (layer "B.Cu") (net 4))
 (segment (start 118.06 122.286998) (end 120.6 119.746998) (width 0.25) (layer "B.Cu") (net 4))
 (segment (start 118.06 126.425001) (end 118.06 122.286998) (width 0.25) (layer "B.Cu") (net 4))
 (segment (start 121.65 121.8) (end 119.63 121.8) (width 0.25) (layer "F.Cu") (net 6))
 (segment (start 119.63 121.8) (end 119.6 121.77) (width 0.25) (layer "F.Cu") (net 6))
 (segment (start 119.6 116.494988) (end 117.6 118.494988) (width 0.25) (layer "F.Cu") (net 7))
 (segment (start 117.6 120.17) (end 117.6 120.82) (width 0.25) (layer "F.Cu") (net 7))
 (segment (start 120 111.4) (end 119.6 111.8) (width 0.25) (layer "F.Cu") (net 7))
 (segment (start 120 109.4825) (end 120 111.4) (width 0.25) (layer "F.Cu") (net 7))
 (segment (start 117.6 118.494988) (end 117.6 120.17) (width 0.25) (layer "F.Cu") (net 7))
 (segment (start 119.6 111.8) (end 119.6 116.494988) (width 0.25) (layer "F.Cu") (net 7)))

